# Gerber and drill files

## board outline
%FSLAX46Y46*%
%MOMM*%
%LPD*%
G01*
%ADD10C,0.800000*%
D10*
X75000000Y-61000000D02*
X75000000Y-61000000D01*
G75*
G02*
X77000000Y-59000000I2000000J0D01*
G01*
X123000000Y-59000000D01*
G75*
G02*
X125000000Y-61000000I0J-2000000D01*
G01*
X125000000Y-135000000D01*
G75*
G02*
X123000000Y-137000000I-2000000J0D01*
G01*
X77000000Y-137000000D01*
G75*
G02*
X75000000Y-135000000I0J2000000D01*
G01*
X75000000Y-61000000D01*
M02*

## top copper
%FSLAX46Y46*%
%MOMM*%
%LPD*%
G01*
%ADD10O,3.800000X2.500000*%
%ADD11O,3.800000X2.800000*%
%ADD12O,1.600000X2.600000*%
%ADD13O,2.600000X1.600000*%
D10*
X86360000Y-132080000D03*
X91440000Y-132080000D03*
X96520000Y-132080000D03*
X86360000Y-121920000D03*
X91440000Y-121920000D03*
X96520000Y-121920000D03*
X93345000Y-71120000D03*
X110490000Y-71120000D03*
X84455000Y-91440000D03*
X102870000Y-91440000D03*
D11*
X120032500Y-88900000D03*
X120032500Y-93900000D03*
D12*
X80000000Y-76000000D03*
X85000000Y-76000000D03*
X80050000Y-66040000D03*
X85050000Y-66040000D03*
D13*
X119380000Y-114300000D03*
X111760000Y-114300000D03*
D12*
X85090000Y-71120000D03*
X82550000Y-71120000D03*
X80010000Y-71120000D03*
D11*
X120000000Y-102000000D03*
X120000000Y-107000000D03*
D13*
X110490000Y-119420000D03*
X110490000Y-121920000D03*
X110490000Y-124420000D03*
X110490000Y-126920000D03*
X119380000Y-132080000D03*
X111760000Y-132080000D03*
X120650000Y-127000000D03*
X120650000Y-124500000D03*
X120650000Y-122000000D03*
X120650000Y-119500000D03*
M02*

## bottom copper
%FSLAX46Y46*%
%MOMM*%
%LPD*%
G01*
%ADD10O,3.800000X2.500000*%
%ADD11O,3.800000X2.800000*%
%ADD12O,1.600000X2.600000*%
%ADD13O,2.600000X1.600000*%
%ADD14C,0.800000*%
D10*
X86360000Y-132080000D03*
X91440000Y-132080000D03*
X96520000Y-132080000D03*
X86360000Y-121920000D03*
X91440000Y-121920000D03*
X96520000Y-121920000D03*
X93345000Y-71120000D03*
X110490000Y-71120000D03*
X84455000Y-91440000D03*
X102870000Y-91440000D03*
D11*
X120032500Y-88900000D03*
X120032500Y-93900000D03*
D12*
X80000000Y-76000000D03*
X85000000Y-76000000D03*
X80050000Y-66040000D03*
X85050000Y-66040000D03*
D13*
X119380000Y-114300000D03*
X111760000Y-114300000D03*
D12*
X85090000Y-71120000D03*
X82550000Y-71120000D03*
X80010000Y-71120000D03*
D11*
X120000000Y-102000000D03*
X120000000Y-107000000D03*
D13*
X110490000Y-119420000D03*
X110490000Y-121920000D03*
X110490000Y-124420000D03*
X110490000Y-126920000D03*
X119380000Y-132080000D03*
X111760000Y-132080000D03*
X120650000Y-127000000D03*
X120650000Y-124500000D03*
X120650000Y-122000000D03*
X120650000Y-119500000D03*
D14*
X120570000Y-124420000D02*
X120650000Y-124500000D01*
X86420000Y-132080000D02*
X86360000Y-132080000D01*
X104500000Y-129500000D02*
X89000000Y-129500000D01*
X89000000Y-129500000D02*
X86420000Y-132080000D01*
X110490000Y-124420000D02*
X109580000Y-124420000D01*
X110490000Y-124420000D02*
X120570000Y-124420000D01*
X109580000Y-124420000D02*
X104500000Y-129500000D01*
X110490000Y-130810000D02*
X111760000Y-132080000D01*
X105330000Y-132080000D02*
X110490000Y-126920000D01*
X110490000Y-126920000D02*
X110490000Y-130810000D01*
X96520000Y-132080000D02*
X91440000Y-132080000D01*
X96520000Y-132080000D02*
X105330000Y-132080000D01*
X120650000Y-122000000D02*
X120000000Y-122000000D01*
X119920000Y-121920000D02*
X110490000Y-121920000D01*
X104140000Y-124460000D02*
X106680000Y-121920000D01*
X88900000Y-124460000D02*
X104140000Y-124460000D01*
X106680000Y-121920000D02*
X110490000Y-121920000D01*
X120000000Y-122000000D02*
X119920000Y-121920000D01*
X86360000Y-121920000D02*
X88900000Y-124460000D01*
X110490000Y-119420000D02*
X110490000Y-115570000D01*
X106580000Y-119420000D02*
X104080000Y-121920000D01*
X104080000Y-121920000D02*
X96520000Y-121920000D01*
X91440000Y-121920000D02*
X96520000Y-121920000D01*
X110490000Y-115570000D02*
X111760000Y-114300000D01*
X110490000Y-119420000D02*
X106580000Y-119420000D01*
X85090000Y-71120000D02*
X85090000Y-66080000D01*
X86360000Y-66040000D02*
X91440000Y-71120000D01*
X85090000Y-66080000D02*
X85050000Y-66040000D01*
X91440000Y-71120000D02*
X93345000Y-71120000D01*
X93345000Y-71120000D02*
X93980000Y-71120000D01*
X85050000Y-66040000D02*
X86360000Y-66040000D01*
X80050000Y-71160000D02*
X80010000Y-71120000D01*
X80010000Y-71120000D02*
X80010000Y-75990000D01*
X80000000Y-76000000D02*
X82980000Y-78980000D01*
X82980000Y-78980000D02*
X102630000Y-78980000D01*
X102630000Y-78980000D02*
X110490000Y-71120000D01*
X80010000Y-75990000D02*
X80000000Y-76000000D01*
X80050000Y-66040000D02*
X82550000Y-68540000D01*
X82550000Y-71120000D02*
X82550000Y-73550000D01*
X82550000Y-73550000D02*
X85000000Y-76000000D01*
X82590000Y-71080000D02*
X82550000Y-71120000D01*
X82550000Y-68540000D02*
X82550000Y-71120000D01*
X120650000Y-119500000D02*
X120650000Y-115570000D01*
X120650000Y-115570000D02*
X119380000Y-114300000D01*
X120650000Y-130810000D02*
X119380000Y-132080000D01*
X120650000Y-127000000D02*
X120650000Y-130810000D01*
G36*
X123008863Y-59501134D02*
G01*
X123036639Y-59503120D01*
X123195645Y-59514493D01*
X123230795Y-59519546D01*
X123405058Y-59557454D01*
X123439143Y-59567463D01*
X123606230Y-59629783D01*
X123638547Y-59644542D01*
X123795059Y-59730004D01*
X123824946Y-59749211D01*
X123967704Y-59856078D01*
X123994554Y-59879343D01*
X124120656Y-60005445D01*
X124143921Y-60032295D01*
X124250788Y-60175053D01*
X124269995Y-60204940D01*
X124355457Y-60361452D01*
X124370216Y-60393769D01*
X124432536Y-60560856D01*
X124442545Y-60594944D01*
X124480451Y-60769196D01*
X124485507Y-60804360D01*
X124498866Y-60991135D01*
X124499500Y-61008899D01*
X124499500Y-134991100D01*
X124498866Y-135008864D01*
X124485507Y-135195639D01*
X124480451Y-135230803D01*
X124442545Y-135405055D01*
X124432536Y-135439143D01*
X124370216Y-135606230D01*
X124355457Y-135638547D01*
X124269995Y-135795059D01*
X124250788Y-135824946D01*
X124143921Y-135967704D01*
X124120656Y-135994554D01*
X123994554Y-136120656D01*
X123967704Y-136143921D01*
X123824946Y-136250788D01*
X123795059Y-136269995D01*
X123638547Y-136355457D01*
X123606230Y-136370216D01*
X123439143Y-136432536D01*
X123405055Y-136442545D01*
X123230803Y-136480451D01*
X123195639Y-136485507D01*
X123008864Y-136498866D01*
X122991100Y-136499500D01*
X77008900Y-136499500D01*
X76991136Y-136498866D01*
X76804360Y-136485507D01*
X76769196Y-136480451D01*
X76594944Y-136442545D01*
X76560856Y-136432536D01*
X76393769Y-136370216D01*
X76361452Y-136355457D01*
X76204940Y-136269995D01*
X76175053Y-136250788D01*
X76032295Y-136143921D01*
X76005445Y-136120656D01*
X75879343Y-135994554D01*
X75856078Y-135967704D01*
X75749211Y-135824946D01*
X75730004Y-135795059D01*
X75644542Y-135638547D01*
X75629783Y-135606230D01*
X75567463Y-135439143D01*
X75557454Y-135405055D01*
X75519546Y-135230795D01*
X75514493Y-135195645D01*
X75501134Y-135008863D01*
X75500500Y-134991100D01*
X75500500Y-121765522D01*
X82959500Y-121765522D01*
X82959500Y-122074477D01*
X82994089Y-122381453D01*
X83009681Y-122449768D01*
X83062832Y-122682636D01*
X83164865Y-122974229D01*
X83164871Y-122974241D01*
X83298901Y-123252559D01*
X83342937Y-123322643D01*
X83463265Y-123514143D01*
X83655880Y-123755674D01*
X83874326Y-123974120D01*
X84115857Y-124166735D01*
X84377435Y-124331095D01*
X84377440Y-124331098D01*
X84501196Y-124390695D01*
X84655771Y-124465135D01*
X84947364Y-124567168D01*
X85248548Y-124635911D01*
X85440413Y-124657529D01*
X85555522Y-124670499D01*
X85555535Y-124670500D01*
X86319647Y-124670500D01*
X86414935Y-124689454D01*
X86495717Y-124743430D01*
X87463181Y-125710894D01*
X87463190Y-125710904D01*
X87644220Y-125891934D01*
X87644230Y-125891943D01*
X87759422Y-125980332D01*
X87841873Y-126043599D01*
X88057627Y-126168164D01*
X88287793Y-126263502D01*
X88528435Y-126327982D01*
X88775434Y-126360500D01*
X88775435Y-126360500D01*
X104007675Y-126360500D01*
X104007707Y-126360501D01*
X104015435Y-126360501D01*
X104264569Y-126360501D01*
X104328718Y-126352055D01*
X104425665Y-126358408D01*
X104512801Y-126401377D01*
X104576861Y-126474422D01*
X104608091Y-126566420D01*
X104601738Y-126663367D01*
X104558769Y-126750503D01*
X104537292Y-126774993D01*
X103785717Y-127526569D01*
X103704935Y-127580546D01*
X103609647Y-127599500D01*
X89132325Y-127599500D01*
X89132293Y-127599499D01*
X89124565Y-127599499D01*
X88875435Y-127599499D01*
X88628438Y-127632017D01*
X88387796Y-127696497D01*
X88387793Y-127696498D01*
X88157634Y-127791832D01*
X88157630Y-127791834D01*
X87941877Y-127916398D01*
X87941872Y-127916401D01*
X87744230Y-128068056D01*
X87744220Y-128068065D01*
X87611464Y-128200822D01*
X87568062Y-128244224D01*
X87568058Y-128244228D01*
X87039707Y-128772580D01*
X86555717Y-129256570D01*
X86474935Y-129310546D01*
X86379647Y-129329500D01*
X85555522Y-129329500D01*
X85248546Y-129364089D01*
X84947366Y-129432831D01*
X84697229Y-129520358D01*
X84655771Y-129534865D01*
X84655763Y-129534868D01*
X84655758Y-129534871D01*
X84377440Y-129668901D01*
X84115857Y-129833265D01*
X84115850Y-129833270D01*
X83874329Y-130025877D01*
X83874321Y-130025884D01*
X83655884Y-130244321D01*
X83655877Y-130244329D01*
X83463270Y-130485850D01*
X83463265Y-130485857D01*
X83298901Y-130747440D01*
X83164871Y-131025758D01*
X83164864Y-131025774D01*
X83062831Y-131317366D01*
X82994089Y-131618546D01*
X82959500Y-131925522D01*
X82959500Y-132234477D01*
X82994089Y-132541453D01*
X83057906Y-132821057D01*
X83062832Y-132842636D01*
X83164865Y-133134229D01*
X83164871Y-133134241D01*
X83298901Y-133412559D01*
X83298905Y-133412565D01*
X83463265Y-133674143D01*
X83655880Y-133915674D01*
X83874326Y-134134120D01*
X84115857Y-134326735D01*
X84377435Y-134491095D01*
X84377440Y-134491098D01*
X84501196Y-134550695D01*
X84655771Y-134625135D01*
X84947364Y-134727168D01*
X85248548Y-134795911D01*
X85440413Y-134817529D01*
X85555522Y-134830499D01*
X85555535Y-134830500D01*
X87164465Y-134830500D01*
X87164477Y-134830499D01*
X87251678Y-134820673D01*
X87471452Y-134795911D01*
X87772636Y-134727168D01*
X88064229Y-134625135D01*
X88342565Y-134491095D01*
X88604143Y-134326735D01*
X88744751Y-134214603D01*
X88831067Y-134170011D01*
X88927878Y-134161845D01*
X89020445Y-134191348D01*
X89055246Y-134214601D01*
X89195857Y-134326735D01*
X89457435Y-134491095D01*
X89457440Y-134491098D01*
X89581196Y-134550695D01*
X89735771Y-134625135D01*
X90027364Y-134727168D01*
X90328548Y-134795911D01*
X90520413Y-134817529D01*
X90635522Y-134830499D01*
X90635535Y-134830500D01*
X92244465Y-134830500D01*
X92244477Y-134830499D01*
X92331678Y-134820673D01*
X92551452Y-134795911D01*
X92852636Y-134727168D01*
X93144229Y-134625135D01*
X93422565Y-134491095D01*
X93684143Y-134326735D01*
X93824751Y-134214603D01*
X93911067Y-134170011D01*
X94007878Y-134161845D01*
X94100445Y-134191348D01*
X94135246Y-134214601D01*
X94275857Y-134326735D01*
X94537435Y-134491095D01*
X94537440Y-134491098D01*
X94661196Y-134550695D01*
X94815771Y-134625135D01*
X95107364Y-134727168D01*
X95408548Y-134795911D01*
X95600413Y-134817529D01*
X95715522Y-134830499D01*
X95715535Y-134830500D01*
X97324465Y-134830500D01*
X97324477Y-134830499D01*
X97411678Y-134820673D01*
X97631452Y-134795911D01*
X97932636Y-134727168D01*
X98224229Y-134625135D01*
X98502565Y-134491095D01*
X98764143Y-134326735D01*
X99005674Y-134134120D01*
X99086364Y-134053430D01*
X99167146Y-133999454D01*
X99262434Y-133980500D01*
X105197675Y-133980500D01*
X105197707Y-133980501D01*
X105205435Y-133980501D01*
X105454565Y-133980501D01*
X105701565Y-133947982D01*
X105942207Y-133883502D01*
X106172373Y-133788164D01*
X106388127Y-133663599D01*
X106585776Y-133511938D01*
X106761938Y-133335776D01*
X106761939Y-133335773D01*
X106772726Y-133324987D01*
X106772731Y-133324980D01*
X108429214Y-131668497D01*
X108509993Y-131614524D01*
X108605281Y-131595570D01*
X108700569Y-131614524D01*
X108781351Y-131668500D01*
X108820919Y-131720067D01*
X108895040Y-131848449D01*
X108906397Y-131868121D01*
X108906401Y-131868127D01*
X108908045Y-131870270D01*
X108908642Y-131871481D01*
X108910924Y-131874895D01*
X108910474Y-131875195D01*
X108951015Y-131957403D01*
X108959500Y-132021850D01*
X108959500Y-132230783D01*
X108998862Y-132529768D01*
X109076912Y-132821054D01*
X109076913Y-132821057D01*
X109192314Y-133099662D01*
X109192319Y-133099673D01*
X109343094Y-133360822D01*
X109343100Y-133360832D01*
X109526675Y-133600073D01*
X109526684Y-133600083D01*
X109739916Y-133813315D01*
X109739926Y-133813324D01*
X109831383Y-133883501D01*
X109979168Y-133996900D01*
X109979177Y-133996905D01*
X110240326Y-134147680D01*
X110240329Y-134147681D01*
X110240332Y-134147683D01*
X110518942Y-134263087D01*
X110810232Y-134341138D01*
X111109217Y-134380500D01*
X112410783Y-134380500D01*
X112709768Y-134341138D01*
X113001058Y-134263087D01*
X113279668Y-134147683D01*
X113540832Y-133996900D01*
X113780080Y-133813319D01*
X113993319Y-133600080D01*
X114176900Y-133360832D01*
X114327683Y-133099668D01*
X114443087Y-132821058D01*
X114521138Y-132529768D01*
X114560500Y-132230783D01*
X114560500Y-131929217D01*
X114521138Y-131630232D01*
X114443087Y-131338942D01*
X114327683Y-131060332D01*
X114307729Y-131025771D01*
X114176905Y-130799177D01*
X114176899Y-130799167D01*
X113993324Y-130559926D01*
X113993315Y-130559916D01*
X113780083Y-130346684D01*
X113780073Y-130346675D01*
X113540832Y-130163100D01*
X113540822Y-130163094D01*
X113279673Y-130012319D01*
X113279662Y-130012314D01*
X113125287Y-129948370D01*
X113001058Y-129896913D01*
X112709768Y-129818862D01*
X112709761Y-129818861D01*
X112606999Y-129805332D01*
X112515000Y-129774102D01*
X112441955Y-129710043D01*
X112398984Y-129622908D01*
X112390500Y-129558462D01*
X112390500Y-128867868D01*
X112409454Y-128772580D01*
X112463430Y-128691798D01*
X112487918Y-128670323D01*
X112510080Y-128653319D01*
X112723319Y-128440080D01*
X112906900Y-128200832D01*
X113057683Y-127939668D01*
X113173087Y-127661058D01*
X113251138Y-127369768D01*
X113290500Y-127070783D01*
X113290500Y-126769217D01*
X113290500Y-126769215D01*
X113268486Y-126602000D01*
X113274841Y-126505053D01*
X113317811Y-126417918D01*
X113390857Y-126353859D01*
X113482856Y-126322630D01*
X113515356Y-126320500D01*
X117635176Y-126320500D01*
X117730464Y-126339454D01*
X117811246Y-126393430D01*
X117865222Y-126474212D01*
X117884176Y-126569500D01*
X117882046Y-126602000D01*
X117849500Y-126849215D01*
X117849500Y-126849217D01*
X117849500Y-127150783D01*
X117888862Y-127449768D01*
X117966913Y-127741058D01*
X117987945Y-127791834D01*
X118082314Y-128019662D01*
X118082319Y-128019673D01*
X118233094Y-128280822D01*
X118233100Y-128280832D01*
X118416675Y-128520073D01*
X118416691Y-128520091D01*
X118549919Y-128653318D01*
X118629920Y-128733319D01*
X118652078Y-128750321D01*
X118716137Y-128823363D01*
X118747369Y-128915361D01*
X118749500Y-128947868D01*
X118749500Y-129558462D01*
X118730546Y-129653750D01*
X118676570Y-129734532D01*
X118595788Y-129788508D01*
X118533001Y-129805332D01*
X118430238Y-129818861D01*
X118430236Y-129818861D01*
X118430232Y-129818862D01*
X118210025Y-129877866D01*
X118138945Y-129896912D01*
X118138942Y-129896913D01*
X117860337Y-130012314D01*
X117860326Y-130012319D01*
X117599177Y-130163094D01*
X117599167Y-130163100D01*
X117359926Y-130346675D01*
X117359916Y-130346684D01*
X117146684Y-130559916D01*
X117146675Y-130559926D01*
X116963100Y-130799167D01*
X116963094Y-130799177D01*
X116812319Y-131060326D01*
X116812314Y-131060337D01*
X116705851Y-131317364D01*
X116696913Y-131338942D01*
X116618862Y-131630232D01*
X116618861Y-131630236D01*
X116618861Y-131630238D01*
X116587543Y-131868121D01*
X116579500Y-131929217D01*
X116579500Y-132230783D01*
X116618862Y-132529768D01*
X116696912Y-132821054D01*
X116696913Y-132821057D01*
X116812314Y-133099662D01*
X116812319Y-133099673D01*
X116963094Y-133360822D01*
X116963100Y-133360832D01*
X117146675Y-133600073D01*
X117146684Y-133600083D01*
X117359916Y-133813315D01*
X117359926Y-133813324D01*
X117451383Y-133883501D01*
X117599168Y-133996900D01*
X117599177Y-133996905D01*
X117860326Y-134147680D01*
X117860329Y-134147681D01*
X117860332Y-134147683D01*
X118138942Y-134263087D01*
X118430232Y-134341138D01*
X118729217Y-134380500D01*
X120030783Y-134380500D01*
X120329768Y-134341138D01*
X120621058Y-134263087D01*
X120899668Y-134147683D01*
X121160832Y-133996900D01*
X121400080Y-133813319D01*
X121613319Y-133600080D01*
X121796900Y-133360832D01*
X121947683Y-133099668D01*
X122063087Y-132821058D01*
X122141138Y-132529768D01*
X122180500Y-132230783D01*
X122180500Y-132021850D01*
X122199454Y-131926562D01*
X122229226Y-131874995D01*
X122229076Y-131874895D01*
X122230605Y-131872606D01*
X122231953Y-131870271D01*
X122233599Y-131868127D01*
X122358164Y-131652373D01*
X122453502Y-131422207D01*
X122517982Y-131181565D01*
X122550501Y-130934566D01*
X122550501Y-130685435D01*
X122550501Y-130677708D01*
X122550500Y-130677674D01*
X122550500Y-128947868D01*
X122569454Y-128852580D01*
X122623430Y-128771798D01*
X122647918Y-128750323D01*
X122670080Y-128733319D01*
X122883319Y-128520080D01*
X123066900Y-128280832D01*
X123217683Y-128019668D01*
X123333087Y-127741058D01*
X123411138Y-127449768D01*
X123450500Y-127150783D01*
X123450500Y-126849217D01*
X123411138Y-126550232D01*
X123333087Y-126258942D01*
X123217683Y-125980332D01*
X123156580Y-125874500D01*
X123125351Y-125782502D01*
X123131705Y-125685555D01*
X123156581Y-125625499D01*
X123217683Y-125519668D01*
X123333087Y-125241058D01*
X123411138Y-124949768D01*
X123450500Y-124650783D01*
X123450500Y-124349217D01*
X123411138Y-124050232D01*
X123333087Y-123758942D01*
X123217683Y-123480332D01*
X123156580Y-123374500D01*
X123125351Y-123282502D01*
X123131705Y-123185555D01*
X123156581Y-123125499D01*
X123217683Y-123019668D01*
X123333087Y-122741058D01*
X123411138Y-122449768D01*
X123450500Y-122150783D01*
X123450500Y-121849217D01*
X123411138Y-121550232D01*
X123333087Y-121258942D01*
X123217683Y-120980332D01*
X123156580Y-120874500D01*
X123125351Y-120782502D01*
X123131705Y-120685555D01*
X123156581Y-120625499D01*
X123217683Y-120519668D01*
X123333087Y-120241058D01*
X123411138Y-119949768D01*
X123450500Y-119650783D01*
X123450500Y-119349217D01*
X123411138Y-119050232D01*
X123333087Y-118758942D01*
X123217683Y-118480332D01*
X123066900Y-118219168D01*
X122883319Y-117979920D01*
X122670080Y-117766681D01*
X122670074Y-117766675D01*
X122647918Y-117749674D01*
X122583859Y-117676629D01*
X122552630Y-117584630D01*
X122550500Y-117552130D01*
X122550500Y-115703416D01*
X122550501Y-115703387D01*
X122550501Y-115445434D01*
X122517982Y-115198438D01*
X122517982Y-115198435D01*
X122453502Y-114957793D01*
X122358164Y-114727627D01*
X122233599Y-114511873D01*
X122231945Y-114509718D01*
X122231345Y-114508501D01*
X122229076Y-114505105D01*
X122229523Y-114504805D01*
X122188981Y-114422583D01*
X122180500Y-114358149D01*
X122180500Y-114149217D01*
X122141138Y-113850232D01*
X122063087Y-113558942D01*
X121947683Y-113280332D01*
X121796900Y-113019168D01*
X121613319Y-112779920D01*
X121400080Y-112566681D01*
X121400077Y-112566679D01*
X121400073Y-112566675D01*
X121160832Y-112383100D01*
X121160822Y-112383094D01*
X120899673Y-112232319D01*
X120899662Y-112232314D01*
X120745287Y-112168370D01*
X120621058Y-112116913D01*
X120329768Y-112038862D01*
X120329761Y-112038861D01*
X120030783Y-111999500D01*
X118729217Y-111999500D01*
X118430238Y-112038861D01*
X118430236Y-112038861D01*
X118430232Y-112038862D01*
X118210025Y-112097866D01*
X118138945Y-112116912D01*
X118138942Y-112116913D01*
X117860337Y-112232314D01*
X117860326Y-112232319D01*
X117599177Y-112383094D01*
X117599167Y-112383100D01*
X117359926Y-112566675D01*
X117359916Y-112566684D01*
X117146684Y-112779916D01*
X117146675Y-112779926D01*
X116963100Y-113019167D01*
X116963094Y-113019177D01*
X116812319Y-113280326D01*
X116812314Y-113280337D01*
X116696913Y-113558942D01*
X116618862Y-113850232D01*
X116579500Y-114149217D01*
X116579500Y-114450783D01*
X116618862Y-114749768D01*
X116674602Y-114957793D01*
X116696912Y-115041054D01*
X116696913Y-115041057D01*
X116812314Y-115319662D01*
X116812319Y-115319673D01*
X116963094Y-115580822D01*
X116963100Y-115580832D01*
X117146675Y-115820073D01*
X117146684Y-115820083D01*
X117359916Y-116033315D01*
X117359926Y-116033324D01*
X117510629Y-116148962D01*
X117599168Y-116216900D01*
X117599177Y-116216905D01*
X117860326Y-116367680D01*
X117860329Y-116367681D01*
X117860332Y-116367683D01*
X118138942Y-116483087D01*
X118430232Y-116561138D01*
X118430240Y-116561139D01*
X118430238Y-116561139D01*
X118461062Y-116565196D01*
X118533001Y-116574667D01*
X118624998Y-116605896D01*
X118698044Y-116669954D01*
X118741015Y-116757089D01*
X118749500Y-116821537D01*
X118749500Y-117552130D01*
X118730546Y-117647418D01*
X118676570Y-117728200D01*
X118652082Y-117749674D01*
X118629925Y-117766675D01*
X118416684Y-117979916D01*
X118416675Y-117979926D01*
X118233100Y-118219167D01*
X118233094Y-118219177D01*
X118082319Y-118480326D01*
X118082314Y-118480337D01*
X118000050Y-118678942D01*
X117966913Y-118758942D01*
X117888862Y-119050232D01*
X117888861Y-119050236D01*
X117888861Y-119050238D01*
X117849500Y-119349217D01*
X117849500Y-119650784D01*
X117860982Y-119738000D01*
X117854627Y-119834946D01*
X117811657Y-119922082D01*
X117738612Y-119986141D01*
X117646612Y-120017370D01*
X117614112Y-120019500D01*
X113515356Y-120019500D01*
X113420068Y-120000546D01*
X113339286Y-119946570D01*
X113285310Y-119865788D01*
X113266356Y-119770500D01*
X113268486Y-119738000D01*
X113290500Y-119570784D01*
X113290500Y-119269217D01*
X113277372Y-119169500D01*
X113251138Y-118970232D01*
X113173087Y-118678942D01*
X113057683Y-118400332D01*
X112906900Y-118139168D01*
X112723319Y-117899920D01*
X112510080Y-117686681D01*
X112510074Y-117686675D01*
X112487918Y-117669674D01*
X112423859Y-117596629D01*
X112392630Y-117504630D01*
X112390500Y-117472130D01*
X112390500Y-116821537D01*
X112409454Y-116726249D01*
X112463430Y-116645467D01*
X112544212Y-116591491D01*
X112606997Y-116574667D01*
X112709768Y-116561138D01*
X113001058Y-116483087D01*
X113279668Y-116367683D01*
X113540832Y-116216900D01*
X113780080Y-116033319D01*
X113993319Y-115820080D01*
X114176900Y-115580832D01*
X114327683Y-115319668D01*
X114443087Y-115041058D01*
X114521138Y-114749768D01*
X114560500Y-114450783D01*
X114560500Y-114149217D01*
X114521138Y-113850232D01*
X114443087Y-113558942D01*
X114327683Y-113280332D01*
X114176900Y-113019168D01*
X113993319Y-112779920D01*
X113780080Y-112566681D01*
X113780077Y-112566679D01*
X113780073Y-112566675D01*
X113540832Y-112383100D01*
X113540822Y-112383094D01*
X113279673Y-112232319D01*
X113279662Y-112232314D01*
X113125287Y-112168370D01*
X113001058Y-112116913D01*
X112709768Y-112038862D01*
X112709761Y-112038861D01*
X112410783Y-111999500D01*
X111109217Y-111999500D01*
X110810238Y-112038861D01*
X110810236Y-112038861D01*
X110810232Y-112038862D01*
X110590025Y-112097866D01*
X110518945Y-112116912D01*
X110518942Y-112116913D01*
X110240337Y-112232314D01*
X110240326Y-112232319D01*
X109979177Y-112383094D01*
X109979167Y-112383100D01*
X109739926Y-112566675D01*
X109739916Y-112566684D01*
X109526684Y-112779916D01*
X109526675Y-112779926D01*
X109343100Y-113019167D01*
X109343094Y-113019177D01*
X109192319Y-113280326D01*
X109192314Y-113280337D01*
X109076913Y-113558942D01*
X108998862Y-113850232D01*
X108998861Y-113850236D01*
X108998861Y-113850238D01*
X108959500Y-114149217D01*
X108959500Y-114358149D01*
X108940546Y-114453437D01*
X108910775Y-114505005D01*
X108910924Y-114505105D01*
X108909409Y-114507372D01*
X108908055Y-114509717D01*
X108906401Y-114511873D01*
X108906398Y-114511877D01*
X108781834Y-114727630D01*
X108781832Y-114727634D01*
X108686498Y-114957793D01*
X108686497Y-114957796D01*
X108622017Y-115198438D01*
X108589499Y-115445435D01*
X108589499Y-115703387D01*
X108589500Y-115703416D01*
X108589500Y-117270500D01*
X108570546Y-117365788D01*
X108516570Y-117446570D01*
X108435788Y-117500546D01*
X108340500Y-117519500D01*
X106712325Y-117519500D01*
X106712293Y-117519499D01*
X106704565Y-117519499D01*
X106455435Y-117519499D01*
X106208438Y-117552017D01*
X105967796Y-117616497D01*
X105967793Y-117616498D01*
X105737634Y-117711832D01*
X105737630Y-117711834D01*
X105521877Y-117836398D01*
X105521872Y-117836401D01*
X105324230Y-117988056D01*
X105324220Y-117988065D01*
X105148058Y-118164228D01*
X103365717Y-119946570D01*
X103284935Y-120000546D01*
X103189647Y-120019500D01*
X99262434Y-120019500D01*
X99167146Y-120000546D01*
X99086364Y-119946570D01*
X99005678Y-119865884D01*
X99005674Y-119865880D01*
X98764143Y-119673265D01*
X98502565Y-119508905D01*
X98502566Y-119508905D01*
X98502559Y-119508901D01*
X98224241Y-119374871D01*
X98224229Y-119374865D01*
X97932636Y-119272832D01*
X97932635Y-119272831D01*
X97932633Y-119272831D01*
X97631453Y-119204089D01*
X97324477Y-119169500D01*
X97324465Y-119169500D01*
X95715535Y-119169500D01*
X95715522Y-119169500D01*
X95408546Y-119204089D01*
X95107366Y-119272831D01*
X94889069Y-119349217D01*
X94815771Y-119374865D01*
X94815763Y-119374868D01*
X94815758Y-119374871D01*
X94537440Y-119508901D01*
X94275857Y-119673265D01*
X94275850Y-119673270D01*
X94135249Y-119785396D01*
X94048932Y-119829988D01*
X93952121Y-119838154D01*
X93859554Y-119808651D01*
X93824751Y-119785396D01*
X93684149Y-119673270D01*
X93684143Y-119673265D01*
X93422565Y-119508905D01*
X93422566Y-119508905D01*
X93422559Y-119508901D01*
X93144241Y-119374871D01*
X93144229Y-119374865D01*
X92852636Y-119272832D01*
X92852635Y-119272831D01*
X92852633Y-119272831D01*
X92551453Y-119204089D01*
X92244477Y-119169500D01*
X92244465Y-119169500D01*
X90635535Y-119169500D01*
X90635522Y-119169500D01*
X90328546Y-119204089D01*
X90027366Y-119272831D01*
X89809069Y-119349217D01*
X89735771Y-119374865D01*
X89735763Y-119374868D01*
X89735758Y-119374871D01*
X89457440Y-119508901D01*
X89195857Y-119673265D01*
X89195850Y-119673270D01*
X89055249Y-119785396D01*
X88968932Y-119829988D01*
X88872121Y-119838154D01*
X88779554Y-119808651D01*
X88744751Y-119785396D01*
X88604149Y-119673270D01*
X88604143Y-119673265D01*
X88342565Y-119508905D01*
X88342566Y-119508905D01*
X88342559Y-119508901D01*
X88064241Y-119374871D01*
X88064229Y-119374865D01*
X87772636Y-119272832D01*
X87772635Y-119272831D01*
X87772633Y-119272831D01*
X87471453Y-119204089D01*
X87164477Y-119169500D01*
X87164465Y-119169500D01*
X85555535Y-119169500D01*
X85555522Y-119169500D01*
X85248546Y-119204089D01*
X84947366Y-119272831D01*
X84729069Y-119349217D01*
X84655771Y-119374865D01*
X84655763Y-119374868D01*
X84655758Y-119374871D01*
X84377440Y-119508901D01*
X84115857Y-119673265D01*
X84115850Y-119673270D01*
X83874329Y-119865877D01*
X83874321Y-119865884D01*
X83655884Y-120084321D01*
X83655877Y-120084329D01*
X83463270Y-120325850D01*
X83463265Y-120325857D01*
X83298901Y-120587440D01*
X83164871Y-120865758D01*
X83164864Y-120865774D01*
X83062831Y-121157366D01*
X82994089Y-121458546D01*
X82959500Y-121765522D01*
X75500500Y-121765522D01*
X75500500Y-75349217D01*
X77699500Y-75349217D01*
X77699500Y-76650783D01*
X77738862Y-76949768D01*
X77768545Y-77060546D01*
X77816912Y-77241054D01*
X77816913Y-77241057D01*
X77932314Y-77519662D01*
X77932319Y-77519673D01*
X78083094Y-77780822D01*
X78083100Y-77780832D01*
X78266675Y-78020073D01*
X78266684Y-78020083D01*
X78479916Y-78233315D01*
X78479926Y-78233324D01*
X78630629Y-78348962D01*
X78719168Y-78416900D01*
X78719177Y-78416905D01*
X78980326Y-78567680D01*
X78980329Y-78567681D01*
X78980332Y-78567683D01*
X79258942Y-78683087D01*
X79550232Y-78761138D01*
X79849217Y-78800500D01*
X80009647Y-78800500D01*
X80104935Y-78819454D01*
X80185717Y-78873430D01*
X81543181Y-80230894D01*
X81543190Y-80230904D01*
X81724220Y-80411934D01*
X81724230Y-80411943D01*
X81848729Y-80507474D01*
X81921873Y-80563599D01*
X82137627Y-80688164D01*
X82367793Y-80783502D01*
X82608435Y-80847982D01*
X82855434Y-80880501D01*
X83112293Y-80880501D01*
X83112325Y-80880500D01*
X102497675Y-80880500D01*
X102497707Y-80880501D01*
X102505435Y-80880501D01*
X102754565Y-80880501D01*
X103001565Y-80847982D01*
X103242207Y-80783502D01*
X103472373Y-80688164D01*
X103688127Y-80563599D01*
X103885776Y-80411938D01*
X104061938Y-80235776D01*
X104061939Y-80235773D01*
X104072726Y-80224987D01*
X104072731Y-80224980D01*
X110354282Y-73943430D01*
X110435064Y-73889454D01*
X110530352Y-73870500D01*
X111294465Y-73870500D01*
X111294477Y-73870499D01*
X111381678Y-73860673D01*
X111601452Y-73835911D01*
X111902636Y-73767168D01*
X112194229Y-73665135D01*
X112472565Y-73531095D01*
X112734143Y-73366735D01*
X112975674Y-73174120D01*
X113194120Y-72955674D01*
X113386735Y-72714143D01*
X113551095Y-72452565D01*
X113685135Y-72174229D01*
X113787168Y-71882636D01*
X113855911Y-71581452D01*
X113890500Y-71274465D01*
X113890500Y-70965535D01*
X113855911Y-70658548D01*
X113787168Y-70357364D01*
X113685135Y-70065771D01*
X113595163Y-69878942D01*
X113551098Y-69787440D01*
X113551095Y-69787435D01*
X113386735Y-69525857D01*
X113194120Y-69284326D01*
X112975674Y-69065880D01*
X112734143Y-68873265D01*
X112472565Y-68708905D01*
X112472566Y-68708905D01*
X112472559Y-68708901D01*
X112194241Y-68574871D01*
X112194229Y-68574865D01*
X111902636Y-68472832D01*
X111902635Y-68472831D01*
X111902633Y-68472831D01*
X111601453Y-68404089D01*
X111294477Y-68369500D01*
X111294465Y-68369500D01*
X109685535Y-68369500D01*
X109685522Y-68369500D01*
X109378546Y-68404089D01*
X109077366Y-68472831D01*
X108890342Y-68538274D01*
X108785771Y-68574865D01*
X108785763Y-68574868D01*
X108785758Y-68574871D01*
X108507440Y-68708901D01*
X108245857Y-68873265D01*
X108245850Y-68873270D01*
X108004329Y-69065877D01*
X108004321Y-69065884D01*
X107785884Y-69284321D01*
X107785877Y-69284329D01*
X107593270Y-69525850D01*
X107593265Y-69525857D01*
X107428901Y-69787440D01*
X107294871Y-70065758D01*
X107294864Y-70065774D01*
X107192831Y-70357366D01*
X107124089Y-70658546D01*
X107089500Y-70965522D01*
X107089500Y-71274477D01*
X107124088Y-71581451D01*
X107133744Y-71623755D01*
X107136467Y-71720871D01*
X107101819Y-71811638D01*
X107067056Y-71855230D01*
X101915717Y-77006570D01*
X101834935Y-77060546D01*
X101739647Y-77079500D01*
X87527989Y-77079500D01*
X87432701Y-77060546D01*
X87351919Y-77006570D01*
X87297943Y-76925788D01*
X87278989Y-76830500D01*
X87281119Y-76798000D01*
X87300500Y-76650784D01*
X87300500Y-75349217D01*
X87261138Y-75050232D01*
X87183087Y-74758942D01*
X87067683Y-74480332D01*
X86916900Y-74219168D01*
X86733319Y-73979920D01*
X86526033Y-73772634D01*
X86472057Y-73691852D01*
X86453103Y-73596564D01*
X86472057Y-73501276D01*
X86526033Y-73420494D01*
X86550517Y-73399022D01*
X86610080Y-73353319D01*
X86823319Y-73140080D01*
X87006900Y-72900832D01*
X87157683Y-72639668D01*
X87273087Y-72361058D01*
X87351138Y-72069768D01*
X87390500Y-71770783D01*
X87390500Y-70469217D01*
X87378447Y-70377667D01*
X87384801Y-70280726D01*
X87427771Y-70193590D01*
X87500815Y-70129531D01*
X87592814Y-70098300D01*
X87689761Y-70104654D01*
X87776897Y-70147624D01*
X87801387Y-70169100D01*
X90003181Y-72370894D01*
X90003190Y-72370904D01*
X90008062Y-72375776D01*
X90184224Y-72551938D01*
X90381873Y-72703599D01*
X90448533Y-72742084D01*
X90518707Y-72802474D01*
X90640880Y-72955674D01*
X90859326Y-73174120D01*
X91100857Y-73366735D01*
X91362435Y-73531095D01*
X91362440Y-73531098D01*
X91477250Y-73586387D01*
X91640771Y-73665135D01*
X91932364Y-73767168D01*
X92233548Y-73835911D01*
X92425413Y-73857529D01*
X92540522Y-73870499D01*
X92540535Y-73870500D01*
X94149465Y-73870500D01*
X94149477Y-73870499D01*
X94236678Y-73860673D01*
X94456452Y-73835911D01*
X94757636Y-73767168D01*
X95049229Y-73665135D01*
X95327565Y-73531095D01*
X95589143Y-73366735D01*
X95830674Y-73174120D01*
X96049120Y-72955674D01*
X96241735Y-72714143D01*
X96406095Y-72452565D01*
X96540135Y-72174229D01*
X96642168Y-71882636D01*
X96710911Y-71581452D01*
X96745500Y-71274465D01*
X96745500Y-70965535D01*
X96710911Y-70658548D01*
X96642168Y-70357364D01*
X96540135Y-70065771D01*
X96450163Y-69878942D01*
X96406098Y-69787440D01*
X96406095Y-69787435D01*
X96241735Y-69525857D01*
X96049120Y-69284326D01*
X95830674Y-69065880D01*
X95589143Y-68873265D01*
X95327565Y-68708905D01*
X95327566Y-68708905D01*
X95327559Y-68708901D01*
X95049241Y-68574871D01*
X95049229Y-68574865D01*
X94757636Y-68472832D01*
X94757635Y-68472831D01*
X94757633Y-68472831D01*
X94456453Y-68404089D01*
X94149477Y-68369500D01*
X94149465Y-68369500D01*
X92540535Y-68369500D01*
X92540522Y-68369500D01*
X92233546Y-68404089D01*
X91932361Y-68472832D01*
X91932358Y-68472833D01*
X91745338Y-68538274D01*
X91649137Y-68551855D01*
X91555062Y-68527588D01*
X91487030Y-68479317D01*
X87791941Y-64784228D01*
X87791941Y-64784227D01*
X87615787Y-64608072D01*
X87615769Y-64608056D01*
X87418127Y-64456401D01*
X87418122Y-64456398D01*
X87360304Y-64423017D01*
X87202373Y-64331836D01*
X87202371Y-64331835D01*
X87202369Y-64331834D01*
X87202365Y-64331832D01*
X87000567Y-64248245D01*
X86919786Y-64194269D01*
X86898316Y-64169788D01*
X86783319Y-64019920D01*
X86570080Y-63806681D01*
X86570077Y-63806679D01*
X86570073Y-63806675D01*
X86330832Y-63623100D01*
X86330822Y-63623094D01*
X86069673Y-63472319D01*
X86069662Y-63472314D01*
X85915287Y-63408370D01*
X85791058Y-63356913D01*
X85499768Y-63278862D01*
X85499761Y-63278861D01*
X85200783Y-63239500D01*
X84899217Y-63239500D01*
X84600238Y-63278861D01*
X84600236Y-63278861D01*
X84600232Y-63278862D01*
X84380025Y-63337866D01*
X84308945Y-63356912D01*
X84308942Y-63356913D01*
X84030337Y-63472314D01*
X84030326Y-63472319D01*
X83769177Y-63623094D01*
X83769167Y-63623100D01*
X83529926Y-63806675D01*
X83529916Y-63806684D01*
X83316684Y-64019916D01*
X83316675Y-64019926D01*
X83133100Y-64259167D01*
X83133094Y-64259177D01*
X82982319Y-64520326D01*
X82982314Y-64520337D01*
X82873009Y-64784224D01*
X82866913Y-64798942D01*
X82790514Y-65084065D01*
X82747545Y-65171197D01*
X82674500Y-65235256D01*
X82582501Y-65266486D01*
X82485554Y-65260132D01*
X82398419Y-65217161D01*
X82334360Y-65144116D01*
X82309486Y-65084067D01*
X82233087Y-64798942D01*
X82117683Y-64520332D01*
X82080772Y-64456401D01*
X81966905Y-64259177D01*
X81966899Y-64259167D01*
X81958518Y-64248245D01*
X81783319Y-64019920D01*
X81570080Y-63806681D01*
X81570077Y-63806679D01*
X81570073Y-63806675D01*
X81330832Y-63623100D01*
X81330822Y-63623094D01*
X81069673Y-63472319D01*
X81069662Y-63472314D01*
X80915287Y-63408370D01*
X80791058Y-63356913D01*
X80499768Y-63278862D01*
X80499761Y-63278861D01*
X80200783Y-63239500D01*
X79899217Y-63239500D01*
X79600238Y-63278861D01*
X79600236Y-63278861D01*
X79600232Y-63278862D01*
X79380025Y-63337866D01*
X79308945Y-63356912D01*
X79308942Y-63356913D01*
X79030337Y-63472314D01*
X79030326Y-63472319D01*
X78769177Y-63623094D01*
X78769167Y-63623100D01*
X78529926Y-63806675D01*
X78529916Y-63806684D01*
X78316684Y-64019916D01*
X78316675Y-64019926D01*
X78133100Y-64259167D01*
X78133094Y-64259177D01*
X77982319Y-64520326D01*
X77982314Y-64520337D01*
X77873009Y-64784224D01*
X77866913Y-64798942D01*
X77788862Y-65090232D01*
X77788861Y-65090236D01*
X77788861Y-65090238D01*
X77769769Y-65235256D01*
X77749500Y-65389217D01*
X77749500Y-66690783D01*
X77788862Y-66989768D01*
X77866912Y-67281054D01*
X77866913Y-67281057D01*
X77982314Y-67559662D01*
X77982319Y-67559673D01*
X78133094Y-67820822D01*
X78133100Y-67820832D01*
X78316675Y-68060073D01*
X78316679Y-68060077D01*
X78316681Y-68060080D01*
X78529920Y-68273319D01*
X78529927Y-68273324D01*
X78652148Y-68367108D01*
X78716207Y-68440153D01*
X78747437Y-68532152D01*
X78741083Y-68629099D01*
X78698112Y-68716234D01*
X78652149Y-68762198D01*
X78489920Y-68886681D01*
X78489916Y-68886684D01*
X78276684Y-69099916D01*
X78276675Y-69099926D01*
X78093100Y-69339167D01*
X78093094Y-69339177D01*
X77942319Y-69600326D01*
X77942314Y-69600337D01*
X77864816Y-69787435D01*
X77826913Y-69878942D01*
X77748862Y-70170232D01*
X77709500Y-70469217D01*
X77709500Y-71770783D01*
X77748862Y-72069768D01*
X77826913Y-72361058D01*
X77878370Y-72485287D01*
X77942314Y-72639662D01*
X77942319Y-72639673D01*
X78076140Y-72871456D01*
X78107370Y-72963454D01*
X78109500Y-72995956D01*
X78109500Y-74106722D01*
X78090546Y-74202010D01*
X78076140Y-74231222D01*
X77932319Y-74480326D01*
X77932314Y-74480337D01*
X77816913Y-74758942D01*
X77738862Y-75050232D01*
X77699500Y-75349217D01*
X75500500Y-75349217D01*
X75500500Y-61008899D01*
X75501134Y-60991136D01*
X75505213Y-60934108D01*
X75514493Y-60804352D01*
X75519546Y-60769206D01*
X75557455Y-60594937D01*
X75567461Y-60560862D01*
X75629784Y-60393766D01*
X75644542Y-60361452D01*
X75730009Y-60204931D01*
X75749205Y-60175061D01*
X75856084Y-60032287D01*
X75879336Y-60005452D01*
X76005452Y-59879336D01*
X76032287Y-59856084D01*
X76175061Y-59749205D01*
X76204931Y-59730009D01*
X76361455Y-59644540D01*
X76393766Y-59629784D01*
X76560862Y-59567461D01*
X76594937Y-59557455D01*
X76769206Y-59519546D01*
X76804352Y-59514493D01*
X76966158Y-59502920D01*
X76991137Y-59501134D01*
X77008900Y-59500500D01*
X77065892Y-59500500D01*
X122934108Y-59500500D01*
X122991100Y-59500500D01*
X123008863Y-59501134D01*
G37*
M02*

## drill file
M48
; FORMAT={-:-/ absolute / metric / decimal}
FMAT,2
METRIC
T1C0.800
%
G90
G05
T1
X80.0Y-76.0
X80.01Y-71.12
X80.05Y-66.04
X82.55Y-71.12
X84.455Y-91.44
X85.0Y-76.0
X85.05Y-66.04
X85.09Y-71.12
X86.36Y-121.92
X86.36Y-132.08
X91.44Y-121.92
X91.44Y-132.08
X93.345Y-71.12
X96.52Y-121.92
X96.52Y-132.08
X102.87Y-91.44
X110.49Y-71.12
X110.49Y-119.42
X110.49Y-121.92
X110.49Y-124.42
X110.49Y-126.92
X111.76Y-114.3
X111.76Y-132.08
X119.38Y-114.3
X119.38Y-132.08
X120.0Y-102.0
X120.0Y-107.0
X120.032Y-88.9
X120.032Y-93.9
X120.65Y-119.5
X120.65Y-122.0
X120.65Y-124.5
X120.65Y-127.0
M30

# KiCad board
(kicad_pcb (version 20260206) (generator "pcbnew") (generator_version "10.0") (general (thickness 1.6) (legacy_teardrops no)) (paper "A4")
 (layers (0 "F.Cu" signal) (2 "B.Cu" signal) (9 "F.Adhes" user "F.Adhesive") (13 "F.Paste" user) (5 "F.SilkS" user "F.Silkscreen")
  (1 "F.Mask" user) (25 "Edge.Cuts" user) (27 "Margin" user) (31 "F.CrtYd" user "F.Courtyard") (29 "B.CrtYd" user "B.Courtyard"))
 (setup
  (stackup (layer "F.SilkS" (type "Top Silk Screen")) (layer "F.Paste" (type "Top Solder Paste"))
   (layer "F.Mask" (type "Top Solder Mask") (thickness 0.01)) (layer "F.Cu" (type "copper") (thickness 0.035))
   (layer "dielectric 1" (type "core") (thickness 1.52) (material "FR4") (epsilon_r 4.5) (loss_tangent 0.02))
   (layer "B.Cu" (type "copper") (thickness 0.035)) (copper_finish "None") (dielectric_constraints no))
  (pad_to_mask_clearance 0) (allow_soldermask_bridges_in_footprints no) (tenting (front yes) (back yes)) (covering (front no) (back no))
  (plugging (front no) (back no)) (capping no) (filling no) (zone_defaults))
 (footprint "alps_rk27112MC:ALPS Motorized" (layer "F.Cu") (at 91.44 96.52 180)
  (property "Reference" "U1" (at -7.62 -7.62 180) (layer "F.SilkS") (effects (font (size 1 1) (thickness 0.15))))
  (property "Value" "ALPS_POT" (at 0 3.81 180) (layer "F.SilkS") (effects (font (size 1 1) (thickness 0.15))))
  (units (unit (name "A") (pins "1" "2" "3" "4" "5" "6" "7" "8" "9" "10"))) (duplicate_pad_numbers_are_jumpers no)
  (pad "1" thru_hole oval (at 5.08 -35.56 180) (size 3.8 2.5) (drill 0.8) (layers "*.Cu" "*.Mask" "F.SilkS") (remove_unused_layers no)
   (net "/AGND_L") (thermal_bridge_angle 45))
  (pad "2" thru_hole oval (at 0 -35.56 180) (size 3.8 2.5) (drill 0.8) (layers "*.Cu" "*.Mask" "F.SilkS") (remove_unused_layers no)
   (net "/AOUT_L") (thermal_bridge_angle 45))
  (pad "3" thru_hole oval (at -5.08 -35.56 180) (size 3.8 2.5) (drill 0.8) (layers "*.Cu" "*.Mask" "F.SilkS") (remove_unused_layers no)
   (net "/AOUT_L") (thermal_bridge_angle 45))
  (pad "4" thru_hole oval (at 5.08 -25.4 180) (size 3.8 2.5) (drill 0.8) (layers "*.Cu" "*.Mask" "F.SilkS") (remove_unused_layers no)
   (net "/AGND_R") (thermal_bridge_angle 45))
  (pad "5" thru_hole oval (at 0 -25.4 180) (size 3.8 2.5) (drill 0.8) (layers "*.Cu" "*.Mask" "F.SilkS") (remove_unused_layers no)
   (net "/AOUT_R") (thermal_bridge_angle 45))
  (pad "6" thru_hole oval (at -5.08 -25.4 180) (size 3.8 2.5) (drill 0.8) (layers "*.Cu" "*.Mask" "F.SilkS") (remove_unused_layers no)
   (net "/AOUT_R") (thermal_bridge_angle 45))
  (pad "7" thru_hole oval (at -1.905 25.4 180) (size 3.8 2.5) (drill 0.8) (layers "*.Cu" "*.Mask" "F.SilkS") (remove_unused_layers no)
   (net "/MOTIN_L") (thermal_bridge_angle 45))
  (pad "8" thru_hole oval (at -19.05 25.4 180) (size 3.8 2.5) (drill 0.8) (layers "*.Cu" "*.Mask" "F.SilkS") (remove_unused_layers no)
   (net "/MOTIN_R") (thermal_bridge_angle 45))
  (pad "9" thru_hole oval (at 6.985 5.08 180) (size 3.8 2.5) (drill 0.8) (layers "*.Cu" "*.Mask" "F.SilkS") (remove_unused_layers no)
   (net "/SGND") (thermal_bridge_angle 45))
  (pad "10" thru_hole oval (at -11.43 5.08 180) (size 3.8 2.5) (drill 0.8) (layers "*.Cu" "*.Mask" "F.SilkS") (remove_unused_layers no)
   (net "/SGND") (thermal_bridge_angle 45)))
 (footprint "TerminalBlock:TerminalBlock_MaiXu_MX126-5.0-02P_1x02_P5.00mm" (layer "F.Cu") (at 120.0325 88.9 -90)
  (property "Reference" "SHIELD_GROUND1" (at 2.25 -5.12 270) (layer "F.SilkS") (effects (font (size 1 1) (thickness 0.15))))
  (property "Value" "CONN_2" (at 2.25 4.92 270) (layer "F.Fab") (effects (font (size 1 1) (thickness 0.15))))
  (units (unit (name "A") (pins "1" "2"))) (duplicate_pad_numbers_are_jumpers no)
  (pad "1" thru_hole oval (at 0 0) (size 3.8 2.8) (drill 0.8) (layers "*.Cu" "*.Mask") (remove_unused_layers no) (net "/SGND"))
  (pad "2" thru_hole oval (at 5 0) (size 3.8 2.8) (drill 0.8) (layers "*.Cu" "*.Mask") (remove_unused_layers no) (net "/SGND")))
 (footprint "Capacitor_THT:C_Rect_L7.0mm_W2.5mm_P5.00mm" (layer "F.Cu") (at 80 76)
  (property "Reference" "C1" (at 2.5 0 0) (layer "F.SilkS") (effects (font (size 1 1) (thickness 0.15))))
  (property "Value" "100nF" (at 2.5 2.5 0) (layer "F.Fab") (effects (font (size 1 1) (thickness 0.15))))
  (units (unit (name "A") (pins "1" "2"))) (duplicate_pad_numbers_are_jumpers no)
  (pad "1" thru_hole oval (at 0 0 90) (size 2.6 1.6) (drill 0.8) (layers "*.Cu" "*.Mask") (remove_unused_layers no) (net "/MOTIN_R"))
  (pad "2" thru_hole oval (at 5 0 90) (size 2.6 1.6) (drill 0.8) (layers "*.Cu" "*.Mask") (remove_unused_layers no) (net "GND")))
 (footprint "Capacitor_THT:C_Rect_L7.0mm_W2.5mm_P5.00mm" (layer "F.Cu") (at 80.05 66.04)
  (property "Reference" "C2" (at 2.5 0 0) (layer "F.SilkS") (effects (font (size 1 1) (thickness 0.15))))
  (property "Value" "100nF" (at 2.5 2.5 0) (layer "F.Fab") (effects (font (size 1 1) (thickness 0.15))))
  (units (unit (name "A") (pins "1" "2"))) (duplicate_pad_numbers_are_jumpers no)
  (pad "1" thru_hole oval (at 0 0 90) (size 2.6 1.6) (drill 0.8) (layers "*.Cu" "*.Mask") (remove_unused_layers no) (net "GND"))
  (pad "2" thru_hole oval (at 5 0 90) (size 2.6 1.6) (drill 0.8) (layers "*.Cu" "*.Mask") (remove_unused_layers no) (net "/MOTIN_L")))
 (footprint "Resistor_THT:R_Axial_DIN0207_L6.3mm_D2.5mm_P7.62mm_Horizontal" (layer "F.Cu") (at 119.38 114.3 180)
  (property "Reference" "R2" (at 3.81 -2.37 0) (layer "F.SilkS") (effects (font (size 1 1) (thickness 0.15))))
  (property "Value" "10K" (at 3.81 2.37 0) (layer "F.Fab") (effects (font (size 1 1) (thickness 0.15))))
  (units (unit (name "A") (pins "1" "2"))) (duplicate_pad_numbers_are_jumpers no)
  (pad "1" thru_hole oval (at 0 0 180) (size 2.6 1.6) (drill 0.8) (layers "*.Cu" "*.Mask") (remove_unused_layers no) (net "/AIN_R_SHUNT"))
  (pad "2" thru_hole oval (at 7.62 0 180) (size 2.6 1.6) (drill 0.8) (layers "*.Cu" "*.Mask") (remove_unused_layers no) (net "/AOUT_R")))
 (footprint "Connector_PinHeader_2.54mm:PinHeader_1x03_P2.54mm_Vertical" (layer "F.Cu") (at 85.09 71.12 -90)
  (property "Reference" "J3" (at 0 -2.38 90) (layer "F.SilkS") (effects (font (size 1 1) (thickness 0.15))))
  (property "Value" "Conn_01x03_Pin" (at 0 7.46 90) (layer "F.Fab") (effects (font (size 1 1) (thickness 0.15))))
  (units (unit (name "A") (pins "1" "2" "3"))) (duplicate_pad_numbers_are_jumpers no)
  (pad "1" thru_hole oval (at 0 0 270) (size 2.6 1.6) (drill 0.8) (layers "*.Cu" "*.Mask") (remove_unused_layers no) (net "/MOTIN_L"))
  (pad "2" thru_hole oval (at 0 2.54 270) (size 2.6 1.6) (drill 0.8) (layers "*.Cu" "*.Mask") (remove_unused_layers no) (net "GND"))
  (pad "3" thru_hole oval (at 0 5.08 270) (size 2.6 1.6) (drill 0.8) (layers "*.Cu" "*.Mask") (remove_unused_layers no) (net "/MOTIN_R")))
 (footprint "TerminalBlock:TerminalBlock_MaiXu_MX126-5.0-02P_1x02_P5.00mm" (layer "F.Cu") (at 120 102 -90)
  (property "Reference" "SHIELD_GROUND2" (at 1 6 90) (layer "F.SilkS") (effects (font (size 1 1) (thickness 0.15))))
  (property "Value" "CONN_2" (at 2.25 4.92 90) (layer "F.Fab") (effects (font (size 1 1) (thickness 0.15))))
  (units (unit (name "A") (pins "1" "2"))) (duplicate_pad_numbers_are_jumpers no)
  (pad "1" thru_hole oval (at 0 0) (size 3.8 2.8) (drill 0.8) (layers "*.Cu" "*.Mask") (remove_unused_layers no) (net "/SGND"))
  (pad "2" thru_hole oval (at 5 0) (size 3.8 2.8) (drill 0.8) (layers "*.Cu" "*.Mask") (remove_unused_layers no) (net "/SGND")))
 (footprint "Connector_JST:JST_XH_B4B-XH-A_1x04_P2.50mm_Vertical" (layer "F.Cu") (at 110.49 119.42 -90)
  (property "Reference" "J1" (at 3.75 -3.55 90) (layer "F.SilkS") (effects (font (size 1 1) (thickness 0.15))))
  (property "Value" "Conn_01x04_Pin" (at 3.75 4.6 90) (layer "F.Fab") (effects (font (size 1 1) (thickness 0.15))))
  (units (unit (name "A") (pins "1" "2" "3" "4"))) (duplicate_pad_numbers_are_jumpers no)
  (pad "1" thru_hole oval (at 0 0) (size 2.6 1.6) (drill 0.8) (layers "*.Cu" "*.Mask") (remove_unused_layers no) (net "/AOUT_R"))
  (pad "2" thru_hole oval (at 2.5 0) (size 2.6 1.6) (drill 0.8) (layers "*.Cu" "*.Mask") (remove_unused_layers no) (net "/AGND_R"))
  (pad "3" thru_hole oval (at 5 0) (size 2.6 1.6) (drill 0.8) (layers "*.Cu" "*.Mask") (remove_unused_layers no) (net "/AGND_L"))
  (pad "4" thru_hole oval (at 7.5 0) (size 2.6 1.6) (drill 0.8) (layers "*.Cu" "*.Mask") (remove_unused_layers no) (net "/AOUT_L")))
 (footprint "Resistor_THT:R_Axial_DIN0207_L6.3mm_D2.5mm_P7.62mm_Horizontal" (layer "F.Cu") (at 119.38 132.08 180)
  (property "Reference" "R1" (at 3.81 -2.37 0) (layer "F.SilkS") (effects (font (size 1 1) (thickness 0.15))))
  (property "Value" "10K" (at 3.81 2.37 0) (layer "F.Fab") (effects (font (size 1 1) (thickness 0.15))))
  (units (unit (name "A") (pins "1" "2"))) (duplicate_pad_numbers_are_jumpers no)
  (pad "1" thru_hole oval (at 0 0 180) (size 2.6 1.6) (drill 0.8) (layers "*.Cu" "*.Mask") (remove_unused_layers no) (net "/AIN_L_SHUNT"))
  (pad "2" thru_hole oval (at 7.62 0 180) (size 2.6 1.6) (drill 0.8) (layers "*.Cu" "*.Mask") (remove_unused_layers no) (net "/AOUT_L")))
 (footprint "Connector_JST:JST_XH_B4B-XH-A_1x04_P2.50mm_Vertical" (layer "F.Cu") (at 120.65 127 90)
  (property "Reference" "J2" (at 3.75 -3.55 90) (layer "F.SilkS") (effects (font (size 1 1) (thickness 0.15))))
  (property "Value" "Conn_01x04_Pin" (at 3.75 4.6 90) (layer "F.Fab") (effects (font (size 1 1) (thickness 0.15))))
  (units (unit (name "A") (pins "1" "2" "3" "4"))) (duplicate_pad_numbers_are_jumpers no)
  (pad "1" thru_hole oval (at 0 0 180) (size 2.6 1.6) (drill 0.8) (layers "*.Cu" "*.Mask") (remove_unused_layers no) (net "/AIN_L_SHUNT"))
  (pad "2" thru_hole oval (at 2.5 0 180) (size 2.6 1.6) (drill 0.8) (layers "*.Cu" "*.Mask") (remove_unused_layers no) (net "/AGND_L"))
  (pad "3" thru_hole oval (at 5 0 180) (size 2.6 1.6) (drill 0.8) (layers "*.Cu" "*.Mask") (remove_unused_layers no) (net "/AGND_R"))
  (pad "4" thru_hole oval (at 7.5 0 180) (size 2.6 1.6) (drill 0.8) (layers "*.Cu" "*.Mask") (remove_unused_layers no) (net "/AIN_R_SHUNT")))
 (gr_rect (start 75 59) (end 125 137) (radius 2) (stroke (width 0.8) (type solid)) (fill no) (layer "Edge.Cuts"))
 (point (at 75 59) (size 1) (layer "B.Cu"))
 (segment (start 120.57 124.42) (end 120.65 124.5) (width 0.8) (layer "B.Cu") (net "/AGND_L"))
 (segment (start 86.42 132.08) (end 86.36 132.08) (width 0.8) (layer "B.Cu") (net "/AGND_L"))
 (segment (start 104.5 129.5) (end 89 129.5) (width 0.8) (layer "B.Cu") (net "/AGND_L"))
 (segment (start 89 129.5) (end 86.42 132.08) (width 0.8) (layer "B.Cu") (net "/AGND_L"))
 (segment (start 110.49 124.42) (end 109.58 124.42) (width 0.8) (layer "B.Cu") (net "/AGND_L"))
 (segment (start 110.49 124.42) (end 120.57 124.42) (width 0.8) (layer "B.Cu") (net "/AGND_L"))
 (segment (start 109.58 124.42) (end 104.5 129.5) (width 0.8) (layer "B.Cu") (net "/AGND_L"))
 (segment (start 110.49 130.81) (end 111.76 132.08) (width 0.8) (layer "B.Cu") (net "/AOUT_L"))
 (segment (start 105.33 132.08) (end 110.49 126.92) (width 0.8) (layer "B.Cu") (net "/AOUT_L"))
 (segment (start 110.49 126.92) (end 110.49 130.81) (width 0.8) (layer "B.Cu") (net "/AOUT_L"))
 (segment (start 96.52 132.08) (end 91.44 132.08) (width 0.8) (layer "B.Cu") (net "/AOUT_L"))
 (segment (start 96.52 132.08) (end 105.33 132.08) (width 0.8) (layer "B.Cu") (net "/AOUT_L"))
 (segment (start 120.65 122) (end 120 122) (width 0.8) (layer "B.Cu") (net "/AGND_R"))
 (segment (start 119.92 121.92) (end 110.49 121.92) (width 0.8) (layer "B.Cu") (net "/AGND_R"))
 (segment (start 104.14 124.46) (end 106.68 121.92) (width 0.8) (layer "B.Cu") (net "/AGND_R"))
 (segment (start 88.9 124.46) (end 104.14 124.46) (width 0.8) (layer "B.Cu") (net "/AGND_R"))
 (segment (start 106.68 121.92) (end 110.49 121.92) (width 0.8) (layer "B.Cu") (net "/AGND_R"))
 (segment (start 120 122) (end 119.92 121.92) (width 0.8) (layer "B.Cu") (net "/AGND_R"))
 (segment (start 86.36 121.92) (end 88.9 124.46) (width 0.8) (layer "B.Cu") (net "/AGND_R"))
 (segment (start 110.49 119.42) (end 110.49 115.57) (width 0.8) (layer "B.Cu") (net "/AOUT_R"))
 (segment (start 106.58 119.42) (end 104.08 121.92) (width 0.8) (layer "B.Cu") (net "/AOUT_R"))
 (segment (start 104.08 121.92) (end 96.52 121.92) (width 0.8) (layer "B.Cu") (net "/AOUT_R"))
 (segment (start 91.44 121.92) (end 96.52 121.92) (width 0.8) (layer "B.Cu") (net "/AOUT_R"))
 (segment (start 110.49 115.57) (end 111.76 114.3) (width 0.8) (layer "B.Cu") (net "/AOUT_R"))
 (segment (start 110.49 119.42) (end 106.58 119.42) (width 0.8) (layer "B.Cu") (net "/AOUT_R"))
 (segment (start 85.09 71.12) (end 85.09 66.08) (width 0.8) (layer "B.Cu") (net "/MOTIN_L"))
 (segment (start 86.36 66.04) (end 91.44 71.12) (width 0.8) (layer "B.Cu") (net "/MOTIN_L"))
 (segment (start 85.09 66.08) (end 85.05 66.04) (width 0.8) (layer "B.Cu") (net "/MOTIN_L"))
 (segment (start 91.44 71.12) (end 93.345 71.12) (width 0.8) (layer "B.Cu") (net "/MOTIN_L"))
 (segment (start 93.345 71.12) (end 93.98 71.12) (width 0.8) (layer "B.Cu") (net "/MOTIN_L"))
 (segment (start 85.05 66.04) (end 86.36 66.04) (width 0.8) (layer "B.Cu") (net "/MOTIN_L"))
 (segment (start 80.05 71.16) (end 80.01 71.12) (width 0.8) (layer "B.Cu") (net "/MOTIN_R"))
 (segment (start 80.01 71.12) (end 80.01 75.99) (width 0.8) (layer "B.Cu") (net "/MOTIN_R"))
 (segment (start 80 76) (end 82.98 78.98) (width 0.8) (layer "B.Cu") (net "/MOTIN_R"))
 (segment (start 82.98 78.98) (end 102.63 78.98) (width 0.8) (layer "B.Cu") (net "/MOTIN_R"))
 (segment (start 102.63 78.98) (end 110.49 71.12) (width 0.8) (layer "B.Cu") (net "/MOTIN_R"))
 (segment (start 80.01 75.99) (end 80 76) (width 0.8) (layer "B.Cu") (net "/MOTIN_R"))
 (segment (start 80.05 66.04) (end 82.55 68.54) (width 0.8) (layer "B.Cu") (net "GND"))
 (segment (start 82.55 71.12) (end 82.55 73.55) (width 0.8) (layer "B.Cu") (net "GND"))
 (segment (start 82.55 73.55) (end 85 76) (width 0.8) (layer "B.Cu") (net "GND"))
 (segment (start 82.59 71.08) (end 82.55 71.12) (width 0.8) (layer "B.Cu") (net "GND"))
 (segment (start 82.55 68.54) (end 82.55 71.12) (width 0.8) (layer "B.Cu") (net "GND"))
 (segment (start 120.65 119.5) (end 120.65 115.57) (width 0.8) (layer "B.Cu") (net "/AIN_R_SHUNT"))
 (segment (start 120.65 115.57) (end 119.38 114.3) (width 0.8) (layer "B.Cu") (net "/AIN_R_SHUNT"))
 (segment (start 120.65 130.81) (end 119.38 132.08) (width 0.8) (layer "B.Cu") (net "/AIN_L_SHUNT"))
 (segment (start 120.65 127) (end 120.65 130.81) (width 0.8) (layer "B.Cu") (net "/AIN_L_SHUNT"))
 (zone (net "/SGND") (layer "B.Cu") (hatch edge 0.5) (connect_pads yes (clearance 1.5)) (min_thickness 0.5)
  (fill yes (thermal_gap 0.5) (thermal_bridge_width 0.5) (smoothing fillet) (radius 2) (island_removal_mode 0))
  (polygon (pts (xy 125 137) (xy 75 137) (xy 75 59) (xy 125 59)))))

